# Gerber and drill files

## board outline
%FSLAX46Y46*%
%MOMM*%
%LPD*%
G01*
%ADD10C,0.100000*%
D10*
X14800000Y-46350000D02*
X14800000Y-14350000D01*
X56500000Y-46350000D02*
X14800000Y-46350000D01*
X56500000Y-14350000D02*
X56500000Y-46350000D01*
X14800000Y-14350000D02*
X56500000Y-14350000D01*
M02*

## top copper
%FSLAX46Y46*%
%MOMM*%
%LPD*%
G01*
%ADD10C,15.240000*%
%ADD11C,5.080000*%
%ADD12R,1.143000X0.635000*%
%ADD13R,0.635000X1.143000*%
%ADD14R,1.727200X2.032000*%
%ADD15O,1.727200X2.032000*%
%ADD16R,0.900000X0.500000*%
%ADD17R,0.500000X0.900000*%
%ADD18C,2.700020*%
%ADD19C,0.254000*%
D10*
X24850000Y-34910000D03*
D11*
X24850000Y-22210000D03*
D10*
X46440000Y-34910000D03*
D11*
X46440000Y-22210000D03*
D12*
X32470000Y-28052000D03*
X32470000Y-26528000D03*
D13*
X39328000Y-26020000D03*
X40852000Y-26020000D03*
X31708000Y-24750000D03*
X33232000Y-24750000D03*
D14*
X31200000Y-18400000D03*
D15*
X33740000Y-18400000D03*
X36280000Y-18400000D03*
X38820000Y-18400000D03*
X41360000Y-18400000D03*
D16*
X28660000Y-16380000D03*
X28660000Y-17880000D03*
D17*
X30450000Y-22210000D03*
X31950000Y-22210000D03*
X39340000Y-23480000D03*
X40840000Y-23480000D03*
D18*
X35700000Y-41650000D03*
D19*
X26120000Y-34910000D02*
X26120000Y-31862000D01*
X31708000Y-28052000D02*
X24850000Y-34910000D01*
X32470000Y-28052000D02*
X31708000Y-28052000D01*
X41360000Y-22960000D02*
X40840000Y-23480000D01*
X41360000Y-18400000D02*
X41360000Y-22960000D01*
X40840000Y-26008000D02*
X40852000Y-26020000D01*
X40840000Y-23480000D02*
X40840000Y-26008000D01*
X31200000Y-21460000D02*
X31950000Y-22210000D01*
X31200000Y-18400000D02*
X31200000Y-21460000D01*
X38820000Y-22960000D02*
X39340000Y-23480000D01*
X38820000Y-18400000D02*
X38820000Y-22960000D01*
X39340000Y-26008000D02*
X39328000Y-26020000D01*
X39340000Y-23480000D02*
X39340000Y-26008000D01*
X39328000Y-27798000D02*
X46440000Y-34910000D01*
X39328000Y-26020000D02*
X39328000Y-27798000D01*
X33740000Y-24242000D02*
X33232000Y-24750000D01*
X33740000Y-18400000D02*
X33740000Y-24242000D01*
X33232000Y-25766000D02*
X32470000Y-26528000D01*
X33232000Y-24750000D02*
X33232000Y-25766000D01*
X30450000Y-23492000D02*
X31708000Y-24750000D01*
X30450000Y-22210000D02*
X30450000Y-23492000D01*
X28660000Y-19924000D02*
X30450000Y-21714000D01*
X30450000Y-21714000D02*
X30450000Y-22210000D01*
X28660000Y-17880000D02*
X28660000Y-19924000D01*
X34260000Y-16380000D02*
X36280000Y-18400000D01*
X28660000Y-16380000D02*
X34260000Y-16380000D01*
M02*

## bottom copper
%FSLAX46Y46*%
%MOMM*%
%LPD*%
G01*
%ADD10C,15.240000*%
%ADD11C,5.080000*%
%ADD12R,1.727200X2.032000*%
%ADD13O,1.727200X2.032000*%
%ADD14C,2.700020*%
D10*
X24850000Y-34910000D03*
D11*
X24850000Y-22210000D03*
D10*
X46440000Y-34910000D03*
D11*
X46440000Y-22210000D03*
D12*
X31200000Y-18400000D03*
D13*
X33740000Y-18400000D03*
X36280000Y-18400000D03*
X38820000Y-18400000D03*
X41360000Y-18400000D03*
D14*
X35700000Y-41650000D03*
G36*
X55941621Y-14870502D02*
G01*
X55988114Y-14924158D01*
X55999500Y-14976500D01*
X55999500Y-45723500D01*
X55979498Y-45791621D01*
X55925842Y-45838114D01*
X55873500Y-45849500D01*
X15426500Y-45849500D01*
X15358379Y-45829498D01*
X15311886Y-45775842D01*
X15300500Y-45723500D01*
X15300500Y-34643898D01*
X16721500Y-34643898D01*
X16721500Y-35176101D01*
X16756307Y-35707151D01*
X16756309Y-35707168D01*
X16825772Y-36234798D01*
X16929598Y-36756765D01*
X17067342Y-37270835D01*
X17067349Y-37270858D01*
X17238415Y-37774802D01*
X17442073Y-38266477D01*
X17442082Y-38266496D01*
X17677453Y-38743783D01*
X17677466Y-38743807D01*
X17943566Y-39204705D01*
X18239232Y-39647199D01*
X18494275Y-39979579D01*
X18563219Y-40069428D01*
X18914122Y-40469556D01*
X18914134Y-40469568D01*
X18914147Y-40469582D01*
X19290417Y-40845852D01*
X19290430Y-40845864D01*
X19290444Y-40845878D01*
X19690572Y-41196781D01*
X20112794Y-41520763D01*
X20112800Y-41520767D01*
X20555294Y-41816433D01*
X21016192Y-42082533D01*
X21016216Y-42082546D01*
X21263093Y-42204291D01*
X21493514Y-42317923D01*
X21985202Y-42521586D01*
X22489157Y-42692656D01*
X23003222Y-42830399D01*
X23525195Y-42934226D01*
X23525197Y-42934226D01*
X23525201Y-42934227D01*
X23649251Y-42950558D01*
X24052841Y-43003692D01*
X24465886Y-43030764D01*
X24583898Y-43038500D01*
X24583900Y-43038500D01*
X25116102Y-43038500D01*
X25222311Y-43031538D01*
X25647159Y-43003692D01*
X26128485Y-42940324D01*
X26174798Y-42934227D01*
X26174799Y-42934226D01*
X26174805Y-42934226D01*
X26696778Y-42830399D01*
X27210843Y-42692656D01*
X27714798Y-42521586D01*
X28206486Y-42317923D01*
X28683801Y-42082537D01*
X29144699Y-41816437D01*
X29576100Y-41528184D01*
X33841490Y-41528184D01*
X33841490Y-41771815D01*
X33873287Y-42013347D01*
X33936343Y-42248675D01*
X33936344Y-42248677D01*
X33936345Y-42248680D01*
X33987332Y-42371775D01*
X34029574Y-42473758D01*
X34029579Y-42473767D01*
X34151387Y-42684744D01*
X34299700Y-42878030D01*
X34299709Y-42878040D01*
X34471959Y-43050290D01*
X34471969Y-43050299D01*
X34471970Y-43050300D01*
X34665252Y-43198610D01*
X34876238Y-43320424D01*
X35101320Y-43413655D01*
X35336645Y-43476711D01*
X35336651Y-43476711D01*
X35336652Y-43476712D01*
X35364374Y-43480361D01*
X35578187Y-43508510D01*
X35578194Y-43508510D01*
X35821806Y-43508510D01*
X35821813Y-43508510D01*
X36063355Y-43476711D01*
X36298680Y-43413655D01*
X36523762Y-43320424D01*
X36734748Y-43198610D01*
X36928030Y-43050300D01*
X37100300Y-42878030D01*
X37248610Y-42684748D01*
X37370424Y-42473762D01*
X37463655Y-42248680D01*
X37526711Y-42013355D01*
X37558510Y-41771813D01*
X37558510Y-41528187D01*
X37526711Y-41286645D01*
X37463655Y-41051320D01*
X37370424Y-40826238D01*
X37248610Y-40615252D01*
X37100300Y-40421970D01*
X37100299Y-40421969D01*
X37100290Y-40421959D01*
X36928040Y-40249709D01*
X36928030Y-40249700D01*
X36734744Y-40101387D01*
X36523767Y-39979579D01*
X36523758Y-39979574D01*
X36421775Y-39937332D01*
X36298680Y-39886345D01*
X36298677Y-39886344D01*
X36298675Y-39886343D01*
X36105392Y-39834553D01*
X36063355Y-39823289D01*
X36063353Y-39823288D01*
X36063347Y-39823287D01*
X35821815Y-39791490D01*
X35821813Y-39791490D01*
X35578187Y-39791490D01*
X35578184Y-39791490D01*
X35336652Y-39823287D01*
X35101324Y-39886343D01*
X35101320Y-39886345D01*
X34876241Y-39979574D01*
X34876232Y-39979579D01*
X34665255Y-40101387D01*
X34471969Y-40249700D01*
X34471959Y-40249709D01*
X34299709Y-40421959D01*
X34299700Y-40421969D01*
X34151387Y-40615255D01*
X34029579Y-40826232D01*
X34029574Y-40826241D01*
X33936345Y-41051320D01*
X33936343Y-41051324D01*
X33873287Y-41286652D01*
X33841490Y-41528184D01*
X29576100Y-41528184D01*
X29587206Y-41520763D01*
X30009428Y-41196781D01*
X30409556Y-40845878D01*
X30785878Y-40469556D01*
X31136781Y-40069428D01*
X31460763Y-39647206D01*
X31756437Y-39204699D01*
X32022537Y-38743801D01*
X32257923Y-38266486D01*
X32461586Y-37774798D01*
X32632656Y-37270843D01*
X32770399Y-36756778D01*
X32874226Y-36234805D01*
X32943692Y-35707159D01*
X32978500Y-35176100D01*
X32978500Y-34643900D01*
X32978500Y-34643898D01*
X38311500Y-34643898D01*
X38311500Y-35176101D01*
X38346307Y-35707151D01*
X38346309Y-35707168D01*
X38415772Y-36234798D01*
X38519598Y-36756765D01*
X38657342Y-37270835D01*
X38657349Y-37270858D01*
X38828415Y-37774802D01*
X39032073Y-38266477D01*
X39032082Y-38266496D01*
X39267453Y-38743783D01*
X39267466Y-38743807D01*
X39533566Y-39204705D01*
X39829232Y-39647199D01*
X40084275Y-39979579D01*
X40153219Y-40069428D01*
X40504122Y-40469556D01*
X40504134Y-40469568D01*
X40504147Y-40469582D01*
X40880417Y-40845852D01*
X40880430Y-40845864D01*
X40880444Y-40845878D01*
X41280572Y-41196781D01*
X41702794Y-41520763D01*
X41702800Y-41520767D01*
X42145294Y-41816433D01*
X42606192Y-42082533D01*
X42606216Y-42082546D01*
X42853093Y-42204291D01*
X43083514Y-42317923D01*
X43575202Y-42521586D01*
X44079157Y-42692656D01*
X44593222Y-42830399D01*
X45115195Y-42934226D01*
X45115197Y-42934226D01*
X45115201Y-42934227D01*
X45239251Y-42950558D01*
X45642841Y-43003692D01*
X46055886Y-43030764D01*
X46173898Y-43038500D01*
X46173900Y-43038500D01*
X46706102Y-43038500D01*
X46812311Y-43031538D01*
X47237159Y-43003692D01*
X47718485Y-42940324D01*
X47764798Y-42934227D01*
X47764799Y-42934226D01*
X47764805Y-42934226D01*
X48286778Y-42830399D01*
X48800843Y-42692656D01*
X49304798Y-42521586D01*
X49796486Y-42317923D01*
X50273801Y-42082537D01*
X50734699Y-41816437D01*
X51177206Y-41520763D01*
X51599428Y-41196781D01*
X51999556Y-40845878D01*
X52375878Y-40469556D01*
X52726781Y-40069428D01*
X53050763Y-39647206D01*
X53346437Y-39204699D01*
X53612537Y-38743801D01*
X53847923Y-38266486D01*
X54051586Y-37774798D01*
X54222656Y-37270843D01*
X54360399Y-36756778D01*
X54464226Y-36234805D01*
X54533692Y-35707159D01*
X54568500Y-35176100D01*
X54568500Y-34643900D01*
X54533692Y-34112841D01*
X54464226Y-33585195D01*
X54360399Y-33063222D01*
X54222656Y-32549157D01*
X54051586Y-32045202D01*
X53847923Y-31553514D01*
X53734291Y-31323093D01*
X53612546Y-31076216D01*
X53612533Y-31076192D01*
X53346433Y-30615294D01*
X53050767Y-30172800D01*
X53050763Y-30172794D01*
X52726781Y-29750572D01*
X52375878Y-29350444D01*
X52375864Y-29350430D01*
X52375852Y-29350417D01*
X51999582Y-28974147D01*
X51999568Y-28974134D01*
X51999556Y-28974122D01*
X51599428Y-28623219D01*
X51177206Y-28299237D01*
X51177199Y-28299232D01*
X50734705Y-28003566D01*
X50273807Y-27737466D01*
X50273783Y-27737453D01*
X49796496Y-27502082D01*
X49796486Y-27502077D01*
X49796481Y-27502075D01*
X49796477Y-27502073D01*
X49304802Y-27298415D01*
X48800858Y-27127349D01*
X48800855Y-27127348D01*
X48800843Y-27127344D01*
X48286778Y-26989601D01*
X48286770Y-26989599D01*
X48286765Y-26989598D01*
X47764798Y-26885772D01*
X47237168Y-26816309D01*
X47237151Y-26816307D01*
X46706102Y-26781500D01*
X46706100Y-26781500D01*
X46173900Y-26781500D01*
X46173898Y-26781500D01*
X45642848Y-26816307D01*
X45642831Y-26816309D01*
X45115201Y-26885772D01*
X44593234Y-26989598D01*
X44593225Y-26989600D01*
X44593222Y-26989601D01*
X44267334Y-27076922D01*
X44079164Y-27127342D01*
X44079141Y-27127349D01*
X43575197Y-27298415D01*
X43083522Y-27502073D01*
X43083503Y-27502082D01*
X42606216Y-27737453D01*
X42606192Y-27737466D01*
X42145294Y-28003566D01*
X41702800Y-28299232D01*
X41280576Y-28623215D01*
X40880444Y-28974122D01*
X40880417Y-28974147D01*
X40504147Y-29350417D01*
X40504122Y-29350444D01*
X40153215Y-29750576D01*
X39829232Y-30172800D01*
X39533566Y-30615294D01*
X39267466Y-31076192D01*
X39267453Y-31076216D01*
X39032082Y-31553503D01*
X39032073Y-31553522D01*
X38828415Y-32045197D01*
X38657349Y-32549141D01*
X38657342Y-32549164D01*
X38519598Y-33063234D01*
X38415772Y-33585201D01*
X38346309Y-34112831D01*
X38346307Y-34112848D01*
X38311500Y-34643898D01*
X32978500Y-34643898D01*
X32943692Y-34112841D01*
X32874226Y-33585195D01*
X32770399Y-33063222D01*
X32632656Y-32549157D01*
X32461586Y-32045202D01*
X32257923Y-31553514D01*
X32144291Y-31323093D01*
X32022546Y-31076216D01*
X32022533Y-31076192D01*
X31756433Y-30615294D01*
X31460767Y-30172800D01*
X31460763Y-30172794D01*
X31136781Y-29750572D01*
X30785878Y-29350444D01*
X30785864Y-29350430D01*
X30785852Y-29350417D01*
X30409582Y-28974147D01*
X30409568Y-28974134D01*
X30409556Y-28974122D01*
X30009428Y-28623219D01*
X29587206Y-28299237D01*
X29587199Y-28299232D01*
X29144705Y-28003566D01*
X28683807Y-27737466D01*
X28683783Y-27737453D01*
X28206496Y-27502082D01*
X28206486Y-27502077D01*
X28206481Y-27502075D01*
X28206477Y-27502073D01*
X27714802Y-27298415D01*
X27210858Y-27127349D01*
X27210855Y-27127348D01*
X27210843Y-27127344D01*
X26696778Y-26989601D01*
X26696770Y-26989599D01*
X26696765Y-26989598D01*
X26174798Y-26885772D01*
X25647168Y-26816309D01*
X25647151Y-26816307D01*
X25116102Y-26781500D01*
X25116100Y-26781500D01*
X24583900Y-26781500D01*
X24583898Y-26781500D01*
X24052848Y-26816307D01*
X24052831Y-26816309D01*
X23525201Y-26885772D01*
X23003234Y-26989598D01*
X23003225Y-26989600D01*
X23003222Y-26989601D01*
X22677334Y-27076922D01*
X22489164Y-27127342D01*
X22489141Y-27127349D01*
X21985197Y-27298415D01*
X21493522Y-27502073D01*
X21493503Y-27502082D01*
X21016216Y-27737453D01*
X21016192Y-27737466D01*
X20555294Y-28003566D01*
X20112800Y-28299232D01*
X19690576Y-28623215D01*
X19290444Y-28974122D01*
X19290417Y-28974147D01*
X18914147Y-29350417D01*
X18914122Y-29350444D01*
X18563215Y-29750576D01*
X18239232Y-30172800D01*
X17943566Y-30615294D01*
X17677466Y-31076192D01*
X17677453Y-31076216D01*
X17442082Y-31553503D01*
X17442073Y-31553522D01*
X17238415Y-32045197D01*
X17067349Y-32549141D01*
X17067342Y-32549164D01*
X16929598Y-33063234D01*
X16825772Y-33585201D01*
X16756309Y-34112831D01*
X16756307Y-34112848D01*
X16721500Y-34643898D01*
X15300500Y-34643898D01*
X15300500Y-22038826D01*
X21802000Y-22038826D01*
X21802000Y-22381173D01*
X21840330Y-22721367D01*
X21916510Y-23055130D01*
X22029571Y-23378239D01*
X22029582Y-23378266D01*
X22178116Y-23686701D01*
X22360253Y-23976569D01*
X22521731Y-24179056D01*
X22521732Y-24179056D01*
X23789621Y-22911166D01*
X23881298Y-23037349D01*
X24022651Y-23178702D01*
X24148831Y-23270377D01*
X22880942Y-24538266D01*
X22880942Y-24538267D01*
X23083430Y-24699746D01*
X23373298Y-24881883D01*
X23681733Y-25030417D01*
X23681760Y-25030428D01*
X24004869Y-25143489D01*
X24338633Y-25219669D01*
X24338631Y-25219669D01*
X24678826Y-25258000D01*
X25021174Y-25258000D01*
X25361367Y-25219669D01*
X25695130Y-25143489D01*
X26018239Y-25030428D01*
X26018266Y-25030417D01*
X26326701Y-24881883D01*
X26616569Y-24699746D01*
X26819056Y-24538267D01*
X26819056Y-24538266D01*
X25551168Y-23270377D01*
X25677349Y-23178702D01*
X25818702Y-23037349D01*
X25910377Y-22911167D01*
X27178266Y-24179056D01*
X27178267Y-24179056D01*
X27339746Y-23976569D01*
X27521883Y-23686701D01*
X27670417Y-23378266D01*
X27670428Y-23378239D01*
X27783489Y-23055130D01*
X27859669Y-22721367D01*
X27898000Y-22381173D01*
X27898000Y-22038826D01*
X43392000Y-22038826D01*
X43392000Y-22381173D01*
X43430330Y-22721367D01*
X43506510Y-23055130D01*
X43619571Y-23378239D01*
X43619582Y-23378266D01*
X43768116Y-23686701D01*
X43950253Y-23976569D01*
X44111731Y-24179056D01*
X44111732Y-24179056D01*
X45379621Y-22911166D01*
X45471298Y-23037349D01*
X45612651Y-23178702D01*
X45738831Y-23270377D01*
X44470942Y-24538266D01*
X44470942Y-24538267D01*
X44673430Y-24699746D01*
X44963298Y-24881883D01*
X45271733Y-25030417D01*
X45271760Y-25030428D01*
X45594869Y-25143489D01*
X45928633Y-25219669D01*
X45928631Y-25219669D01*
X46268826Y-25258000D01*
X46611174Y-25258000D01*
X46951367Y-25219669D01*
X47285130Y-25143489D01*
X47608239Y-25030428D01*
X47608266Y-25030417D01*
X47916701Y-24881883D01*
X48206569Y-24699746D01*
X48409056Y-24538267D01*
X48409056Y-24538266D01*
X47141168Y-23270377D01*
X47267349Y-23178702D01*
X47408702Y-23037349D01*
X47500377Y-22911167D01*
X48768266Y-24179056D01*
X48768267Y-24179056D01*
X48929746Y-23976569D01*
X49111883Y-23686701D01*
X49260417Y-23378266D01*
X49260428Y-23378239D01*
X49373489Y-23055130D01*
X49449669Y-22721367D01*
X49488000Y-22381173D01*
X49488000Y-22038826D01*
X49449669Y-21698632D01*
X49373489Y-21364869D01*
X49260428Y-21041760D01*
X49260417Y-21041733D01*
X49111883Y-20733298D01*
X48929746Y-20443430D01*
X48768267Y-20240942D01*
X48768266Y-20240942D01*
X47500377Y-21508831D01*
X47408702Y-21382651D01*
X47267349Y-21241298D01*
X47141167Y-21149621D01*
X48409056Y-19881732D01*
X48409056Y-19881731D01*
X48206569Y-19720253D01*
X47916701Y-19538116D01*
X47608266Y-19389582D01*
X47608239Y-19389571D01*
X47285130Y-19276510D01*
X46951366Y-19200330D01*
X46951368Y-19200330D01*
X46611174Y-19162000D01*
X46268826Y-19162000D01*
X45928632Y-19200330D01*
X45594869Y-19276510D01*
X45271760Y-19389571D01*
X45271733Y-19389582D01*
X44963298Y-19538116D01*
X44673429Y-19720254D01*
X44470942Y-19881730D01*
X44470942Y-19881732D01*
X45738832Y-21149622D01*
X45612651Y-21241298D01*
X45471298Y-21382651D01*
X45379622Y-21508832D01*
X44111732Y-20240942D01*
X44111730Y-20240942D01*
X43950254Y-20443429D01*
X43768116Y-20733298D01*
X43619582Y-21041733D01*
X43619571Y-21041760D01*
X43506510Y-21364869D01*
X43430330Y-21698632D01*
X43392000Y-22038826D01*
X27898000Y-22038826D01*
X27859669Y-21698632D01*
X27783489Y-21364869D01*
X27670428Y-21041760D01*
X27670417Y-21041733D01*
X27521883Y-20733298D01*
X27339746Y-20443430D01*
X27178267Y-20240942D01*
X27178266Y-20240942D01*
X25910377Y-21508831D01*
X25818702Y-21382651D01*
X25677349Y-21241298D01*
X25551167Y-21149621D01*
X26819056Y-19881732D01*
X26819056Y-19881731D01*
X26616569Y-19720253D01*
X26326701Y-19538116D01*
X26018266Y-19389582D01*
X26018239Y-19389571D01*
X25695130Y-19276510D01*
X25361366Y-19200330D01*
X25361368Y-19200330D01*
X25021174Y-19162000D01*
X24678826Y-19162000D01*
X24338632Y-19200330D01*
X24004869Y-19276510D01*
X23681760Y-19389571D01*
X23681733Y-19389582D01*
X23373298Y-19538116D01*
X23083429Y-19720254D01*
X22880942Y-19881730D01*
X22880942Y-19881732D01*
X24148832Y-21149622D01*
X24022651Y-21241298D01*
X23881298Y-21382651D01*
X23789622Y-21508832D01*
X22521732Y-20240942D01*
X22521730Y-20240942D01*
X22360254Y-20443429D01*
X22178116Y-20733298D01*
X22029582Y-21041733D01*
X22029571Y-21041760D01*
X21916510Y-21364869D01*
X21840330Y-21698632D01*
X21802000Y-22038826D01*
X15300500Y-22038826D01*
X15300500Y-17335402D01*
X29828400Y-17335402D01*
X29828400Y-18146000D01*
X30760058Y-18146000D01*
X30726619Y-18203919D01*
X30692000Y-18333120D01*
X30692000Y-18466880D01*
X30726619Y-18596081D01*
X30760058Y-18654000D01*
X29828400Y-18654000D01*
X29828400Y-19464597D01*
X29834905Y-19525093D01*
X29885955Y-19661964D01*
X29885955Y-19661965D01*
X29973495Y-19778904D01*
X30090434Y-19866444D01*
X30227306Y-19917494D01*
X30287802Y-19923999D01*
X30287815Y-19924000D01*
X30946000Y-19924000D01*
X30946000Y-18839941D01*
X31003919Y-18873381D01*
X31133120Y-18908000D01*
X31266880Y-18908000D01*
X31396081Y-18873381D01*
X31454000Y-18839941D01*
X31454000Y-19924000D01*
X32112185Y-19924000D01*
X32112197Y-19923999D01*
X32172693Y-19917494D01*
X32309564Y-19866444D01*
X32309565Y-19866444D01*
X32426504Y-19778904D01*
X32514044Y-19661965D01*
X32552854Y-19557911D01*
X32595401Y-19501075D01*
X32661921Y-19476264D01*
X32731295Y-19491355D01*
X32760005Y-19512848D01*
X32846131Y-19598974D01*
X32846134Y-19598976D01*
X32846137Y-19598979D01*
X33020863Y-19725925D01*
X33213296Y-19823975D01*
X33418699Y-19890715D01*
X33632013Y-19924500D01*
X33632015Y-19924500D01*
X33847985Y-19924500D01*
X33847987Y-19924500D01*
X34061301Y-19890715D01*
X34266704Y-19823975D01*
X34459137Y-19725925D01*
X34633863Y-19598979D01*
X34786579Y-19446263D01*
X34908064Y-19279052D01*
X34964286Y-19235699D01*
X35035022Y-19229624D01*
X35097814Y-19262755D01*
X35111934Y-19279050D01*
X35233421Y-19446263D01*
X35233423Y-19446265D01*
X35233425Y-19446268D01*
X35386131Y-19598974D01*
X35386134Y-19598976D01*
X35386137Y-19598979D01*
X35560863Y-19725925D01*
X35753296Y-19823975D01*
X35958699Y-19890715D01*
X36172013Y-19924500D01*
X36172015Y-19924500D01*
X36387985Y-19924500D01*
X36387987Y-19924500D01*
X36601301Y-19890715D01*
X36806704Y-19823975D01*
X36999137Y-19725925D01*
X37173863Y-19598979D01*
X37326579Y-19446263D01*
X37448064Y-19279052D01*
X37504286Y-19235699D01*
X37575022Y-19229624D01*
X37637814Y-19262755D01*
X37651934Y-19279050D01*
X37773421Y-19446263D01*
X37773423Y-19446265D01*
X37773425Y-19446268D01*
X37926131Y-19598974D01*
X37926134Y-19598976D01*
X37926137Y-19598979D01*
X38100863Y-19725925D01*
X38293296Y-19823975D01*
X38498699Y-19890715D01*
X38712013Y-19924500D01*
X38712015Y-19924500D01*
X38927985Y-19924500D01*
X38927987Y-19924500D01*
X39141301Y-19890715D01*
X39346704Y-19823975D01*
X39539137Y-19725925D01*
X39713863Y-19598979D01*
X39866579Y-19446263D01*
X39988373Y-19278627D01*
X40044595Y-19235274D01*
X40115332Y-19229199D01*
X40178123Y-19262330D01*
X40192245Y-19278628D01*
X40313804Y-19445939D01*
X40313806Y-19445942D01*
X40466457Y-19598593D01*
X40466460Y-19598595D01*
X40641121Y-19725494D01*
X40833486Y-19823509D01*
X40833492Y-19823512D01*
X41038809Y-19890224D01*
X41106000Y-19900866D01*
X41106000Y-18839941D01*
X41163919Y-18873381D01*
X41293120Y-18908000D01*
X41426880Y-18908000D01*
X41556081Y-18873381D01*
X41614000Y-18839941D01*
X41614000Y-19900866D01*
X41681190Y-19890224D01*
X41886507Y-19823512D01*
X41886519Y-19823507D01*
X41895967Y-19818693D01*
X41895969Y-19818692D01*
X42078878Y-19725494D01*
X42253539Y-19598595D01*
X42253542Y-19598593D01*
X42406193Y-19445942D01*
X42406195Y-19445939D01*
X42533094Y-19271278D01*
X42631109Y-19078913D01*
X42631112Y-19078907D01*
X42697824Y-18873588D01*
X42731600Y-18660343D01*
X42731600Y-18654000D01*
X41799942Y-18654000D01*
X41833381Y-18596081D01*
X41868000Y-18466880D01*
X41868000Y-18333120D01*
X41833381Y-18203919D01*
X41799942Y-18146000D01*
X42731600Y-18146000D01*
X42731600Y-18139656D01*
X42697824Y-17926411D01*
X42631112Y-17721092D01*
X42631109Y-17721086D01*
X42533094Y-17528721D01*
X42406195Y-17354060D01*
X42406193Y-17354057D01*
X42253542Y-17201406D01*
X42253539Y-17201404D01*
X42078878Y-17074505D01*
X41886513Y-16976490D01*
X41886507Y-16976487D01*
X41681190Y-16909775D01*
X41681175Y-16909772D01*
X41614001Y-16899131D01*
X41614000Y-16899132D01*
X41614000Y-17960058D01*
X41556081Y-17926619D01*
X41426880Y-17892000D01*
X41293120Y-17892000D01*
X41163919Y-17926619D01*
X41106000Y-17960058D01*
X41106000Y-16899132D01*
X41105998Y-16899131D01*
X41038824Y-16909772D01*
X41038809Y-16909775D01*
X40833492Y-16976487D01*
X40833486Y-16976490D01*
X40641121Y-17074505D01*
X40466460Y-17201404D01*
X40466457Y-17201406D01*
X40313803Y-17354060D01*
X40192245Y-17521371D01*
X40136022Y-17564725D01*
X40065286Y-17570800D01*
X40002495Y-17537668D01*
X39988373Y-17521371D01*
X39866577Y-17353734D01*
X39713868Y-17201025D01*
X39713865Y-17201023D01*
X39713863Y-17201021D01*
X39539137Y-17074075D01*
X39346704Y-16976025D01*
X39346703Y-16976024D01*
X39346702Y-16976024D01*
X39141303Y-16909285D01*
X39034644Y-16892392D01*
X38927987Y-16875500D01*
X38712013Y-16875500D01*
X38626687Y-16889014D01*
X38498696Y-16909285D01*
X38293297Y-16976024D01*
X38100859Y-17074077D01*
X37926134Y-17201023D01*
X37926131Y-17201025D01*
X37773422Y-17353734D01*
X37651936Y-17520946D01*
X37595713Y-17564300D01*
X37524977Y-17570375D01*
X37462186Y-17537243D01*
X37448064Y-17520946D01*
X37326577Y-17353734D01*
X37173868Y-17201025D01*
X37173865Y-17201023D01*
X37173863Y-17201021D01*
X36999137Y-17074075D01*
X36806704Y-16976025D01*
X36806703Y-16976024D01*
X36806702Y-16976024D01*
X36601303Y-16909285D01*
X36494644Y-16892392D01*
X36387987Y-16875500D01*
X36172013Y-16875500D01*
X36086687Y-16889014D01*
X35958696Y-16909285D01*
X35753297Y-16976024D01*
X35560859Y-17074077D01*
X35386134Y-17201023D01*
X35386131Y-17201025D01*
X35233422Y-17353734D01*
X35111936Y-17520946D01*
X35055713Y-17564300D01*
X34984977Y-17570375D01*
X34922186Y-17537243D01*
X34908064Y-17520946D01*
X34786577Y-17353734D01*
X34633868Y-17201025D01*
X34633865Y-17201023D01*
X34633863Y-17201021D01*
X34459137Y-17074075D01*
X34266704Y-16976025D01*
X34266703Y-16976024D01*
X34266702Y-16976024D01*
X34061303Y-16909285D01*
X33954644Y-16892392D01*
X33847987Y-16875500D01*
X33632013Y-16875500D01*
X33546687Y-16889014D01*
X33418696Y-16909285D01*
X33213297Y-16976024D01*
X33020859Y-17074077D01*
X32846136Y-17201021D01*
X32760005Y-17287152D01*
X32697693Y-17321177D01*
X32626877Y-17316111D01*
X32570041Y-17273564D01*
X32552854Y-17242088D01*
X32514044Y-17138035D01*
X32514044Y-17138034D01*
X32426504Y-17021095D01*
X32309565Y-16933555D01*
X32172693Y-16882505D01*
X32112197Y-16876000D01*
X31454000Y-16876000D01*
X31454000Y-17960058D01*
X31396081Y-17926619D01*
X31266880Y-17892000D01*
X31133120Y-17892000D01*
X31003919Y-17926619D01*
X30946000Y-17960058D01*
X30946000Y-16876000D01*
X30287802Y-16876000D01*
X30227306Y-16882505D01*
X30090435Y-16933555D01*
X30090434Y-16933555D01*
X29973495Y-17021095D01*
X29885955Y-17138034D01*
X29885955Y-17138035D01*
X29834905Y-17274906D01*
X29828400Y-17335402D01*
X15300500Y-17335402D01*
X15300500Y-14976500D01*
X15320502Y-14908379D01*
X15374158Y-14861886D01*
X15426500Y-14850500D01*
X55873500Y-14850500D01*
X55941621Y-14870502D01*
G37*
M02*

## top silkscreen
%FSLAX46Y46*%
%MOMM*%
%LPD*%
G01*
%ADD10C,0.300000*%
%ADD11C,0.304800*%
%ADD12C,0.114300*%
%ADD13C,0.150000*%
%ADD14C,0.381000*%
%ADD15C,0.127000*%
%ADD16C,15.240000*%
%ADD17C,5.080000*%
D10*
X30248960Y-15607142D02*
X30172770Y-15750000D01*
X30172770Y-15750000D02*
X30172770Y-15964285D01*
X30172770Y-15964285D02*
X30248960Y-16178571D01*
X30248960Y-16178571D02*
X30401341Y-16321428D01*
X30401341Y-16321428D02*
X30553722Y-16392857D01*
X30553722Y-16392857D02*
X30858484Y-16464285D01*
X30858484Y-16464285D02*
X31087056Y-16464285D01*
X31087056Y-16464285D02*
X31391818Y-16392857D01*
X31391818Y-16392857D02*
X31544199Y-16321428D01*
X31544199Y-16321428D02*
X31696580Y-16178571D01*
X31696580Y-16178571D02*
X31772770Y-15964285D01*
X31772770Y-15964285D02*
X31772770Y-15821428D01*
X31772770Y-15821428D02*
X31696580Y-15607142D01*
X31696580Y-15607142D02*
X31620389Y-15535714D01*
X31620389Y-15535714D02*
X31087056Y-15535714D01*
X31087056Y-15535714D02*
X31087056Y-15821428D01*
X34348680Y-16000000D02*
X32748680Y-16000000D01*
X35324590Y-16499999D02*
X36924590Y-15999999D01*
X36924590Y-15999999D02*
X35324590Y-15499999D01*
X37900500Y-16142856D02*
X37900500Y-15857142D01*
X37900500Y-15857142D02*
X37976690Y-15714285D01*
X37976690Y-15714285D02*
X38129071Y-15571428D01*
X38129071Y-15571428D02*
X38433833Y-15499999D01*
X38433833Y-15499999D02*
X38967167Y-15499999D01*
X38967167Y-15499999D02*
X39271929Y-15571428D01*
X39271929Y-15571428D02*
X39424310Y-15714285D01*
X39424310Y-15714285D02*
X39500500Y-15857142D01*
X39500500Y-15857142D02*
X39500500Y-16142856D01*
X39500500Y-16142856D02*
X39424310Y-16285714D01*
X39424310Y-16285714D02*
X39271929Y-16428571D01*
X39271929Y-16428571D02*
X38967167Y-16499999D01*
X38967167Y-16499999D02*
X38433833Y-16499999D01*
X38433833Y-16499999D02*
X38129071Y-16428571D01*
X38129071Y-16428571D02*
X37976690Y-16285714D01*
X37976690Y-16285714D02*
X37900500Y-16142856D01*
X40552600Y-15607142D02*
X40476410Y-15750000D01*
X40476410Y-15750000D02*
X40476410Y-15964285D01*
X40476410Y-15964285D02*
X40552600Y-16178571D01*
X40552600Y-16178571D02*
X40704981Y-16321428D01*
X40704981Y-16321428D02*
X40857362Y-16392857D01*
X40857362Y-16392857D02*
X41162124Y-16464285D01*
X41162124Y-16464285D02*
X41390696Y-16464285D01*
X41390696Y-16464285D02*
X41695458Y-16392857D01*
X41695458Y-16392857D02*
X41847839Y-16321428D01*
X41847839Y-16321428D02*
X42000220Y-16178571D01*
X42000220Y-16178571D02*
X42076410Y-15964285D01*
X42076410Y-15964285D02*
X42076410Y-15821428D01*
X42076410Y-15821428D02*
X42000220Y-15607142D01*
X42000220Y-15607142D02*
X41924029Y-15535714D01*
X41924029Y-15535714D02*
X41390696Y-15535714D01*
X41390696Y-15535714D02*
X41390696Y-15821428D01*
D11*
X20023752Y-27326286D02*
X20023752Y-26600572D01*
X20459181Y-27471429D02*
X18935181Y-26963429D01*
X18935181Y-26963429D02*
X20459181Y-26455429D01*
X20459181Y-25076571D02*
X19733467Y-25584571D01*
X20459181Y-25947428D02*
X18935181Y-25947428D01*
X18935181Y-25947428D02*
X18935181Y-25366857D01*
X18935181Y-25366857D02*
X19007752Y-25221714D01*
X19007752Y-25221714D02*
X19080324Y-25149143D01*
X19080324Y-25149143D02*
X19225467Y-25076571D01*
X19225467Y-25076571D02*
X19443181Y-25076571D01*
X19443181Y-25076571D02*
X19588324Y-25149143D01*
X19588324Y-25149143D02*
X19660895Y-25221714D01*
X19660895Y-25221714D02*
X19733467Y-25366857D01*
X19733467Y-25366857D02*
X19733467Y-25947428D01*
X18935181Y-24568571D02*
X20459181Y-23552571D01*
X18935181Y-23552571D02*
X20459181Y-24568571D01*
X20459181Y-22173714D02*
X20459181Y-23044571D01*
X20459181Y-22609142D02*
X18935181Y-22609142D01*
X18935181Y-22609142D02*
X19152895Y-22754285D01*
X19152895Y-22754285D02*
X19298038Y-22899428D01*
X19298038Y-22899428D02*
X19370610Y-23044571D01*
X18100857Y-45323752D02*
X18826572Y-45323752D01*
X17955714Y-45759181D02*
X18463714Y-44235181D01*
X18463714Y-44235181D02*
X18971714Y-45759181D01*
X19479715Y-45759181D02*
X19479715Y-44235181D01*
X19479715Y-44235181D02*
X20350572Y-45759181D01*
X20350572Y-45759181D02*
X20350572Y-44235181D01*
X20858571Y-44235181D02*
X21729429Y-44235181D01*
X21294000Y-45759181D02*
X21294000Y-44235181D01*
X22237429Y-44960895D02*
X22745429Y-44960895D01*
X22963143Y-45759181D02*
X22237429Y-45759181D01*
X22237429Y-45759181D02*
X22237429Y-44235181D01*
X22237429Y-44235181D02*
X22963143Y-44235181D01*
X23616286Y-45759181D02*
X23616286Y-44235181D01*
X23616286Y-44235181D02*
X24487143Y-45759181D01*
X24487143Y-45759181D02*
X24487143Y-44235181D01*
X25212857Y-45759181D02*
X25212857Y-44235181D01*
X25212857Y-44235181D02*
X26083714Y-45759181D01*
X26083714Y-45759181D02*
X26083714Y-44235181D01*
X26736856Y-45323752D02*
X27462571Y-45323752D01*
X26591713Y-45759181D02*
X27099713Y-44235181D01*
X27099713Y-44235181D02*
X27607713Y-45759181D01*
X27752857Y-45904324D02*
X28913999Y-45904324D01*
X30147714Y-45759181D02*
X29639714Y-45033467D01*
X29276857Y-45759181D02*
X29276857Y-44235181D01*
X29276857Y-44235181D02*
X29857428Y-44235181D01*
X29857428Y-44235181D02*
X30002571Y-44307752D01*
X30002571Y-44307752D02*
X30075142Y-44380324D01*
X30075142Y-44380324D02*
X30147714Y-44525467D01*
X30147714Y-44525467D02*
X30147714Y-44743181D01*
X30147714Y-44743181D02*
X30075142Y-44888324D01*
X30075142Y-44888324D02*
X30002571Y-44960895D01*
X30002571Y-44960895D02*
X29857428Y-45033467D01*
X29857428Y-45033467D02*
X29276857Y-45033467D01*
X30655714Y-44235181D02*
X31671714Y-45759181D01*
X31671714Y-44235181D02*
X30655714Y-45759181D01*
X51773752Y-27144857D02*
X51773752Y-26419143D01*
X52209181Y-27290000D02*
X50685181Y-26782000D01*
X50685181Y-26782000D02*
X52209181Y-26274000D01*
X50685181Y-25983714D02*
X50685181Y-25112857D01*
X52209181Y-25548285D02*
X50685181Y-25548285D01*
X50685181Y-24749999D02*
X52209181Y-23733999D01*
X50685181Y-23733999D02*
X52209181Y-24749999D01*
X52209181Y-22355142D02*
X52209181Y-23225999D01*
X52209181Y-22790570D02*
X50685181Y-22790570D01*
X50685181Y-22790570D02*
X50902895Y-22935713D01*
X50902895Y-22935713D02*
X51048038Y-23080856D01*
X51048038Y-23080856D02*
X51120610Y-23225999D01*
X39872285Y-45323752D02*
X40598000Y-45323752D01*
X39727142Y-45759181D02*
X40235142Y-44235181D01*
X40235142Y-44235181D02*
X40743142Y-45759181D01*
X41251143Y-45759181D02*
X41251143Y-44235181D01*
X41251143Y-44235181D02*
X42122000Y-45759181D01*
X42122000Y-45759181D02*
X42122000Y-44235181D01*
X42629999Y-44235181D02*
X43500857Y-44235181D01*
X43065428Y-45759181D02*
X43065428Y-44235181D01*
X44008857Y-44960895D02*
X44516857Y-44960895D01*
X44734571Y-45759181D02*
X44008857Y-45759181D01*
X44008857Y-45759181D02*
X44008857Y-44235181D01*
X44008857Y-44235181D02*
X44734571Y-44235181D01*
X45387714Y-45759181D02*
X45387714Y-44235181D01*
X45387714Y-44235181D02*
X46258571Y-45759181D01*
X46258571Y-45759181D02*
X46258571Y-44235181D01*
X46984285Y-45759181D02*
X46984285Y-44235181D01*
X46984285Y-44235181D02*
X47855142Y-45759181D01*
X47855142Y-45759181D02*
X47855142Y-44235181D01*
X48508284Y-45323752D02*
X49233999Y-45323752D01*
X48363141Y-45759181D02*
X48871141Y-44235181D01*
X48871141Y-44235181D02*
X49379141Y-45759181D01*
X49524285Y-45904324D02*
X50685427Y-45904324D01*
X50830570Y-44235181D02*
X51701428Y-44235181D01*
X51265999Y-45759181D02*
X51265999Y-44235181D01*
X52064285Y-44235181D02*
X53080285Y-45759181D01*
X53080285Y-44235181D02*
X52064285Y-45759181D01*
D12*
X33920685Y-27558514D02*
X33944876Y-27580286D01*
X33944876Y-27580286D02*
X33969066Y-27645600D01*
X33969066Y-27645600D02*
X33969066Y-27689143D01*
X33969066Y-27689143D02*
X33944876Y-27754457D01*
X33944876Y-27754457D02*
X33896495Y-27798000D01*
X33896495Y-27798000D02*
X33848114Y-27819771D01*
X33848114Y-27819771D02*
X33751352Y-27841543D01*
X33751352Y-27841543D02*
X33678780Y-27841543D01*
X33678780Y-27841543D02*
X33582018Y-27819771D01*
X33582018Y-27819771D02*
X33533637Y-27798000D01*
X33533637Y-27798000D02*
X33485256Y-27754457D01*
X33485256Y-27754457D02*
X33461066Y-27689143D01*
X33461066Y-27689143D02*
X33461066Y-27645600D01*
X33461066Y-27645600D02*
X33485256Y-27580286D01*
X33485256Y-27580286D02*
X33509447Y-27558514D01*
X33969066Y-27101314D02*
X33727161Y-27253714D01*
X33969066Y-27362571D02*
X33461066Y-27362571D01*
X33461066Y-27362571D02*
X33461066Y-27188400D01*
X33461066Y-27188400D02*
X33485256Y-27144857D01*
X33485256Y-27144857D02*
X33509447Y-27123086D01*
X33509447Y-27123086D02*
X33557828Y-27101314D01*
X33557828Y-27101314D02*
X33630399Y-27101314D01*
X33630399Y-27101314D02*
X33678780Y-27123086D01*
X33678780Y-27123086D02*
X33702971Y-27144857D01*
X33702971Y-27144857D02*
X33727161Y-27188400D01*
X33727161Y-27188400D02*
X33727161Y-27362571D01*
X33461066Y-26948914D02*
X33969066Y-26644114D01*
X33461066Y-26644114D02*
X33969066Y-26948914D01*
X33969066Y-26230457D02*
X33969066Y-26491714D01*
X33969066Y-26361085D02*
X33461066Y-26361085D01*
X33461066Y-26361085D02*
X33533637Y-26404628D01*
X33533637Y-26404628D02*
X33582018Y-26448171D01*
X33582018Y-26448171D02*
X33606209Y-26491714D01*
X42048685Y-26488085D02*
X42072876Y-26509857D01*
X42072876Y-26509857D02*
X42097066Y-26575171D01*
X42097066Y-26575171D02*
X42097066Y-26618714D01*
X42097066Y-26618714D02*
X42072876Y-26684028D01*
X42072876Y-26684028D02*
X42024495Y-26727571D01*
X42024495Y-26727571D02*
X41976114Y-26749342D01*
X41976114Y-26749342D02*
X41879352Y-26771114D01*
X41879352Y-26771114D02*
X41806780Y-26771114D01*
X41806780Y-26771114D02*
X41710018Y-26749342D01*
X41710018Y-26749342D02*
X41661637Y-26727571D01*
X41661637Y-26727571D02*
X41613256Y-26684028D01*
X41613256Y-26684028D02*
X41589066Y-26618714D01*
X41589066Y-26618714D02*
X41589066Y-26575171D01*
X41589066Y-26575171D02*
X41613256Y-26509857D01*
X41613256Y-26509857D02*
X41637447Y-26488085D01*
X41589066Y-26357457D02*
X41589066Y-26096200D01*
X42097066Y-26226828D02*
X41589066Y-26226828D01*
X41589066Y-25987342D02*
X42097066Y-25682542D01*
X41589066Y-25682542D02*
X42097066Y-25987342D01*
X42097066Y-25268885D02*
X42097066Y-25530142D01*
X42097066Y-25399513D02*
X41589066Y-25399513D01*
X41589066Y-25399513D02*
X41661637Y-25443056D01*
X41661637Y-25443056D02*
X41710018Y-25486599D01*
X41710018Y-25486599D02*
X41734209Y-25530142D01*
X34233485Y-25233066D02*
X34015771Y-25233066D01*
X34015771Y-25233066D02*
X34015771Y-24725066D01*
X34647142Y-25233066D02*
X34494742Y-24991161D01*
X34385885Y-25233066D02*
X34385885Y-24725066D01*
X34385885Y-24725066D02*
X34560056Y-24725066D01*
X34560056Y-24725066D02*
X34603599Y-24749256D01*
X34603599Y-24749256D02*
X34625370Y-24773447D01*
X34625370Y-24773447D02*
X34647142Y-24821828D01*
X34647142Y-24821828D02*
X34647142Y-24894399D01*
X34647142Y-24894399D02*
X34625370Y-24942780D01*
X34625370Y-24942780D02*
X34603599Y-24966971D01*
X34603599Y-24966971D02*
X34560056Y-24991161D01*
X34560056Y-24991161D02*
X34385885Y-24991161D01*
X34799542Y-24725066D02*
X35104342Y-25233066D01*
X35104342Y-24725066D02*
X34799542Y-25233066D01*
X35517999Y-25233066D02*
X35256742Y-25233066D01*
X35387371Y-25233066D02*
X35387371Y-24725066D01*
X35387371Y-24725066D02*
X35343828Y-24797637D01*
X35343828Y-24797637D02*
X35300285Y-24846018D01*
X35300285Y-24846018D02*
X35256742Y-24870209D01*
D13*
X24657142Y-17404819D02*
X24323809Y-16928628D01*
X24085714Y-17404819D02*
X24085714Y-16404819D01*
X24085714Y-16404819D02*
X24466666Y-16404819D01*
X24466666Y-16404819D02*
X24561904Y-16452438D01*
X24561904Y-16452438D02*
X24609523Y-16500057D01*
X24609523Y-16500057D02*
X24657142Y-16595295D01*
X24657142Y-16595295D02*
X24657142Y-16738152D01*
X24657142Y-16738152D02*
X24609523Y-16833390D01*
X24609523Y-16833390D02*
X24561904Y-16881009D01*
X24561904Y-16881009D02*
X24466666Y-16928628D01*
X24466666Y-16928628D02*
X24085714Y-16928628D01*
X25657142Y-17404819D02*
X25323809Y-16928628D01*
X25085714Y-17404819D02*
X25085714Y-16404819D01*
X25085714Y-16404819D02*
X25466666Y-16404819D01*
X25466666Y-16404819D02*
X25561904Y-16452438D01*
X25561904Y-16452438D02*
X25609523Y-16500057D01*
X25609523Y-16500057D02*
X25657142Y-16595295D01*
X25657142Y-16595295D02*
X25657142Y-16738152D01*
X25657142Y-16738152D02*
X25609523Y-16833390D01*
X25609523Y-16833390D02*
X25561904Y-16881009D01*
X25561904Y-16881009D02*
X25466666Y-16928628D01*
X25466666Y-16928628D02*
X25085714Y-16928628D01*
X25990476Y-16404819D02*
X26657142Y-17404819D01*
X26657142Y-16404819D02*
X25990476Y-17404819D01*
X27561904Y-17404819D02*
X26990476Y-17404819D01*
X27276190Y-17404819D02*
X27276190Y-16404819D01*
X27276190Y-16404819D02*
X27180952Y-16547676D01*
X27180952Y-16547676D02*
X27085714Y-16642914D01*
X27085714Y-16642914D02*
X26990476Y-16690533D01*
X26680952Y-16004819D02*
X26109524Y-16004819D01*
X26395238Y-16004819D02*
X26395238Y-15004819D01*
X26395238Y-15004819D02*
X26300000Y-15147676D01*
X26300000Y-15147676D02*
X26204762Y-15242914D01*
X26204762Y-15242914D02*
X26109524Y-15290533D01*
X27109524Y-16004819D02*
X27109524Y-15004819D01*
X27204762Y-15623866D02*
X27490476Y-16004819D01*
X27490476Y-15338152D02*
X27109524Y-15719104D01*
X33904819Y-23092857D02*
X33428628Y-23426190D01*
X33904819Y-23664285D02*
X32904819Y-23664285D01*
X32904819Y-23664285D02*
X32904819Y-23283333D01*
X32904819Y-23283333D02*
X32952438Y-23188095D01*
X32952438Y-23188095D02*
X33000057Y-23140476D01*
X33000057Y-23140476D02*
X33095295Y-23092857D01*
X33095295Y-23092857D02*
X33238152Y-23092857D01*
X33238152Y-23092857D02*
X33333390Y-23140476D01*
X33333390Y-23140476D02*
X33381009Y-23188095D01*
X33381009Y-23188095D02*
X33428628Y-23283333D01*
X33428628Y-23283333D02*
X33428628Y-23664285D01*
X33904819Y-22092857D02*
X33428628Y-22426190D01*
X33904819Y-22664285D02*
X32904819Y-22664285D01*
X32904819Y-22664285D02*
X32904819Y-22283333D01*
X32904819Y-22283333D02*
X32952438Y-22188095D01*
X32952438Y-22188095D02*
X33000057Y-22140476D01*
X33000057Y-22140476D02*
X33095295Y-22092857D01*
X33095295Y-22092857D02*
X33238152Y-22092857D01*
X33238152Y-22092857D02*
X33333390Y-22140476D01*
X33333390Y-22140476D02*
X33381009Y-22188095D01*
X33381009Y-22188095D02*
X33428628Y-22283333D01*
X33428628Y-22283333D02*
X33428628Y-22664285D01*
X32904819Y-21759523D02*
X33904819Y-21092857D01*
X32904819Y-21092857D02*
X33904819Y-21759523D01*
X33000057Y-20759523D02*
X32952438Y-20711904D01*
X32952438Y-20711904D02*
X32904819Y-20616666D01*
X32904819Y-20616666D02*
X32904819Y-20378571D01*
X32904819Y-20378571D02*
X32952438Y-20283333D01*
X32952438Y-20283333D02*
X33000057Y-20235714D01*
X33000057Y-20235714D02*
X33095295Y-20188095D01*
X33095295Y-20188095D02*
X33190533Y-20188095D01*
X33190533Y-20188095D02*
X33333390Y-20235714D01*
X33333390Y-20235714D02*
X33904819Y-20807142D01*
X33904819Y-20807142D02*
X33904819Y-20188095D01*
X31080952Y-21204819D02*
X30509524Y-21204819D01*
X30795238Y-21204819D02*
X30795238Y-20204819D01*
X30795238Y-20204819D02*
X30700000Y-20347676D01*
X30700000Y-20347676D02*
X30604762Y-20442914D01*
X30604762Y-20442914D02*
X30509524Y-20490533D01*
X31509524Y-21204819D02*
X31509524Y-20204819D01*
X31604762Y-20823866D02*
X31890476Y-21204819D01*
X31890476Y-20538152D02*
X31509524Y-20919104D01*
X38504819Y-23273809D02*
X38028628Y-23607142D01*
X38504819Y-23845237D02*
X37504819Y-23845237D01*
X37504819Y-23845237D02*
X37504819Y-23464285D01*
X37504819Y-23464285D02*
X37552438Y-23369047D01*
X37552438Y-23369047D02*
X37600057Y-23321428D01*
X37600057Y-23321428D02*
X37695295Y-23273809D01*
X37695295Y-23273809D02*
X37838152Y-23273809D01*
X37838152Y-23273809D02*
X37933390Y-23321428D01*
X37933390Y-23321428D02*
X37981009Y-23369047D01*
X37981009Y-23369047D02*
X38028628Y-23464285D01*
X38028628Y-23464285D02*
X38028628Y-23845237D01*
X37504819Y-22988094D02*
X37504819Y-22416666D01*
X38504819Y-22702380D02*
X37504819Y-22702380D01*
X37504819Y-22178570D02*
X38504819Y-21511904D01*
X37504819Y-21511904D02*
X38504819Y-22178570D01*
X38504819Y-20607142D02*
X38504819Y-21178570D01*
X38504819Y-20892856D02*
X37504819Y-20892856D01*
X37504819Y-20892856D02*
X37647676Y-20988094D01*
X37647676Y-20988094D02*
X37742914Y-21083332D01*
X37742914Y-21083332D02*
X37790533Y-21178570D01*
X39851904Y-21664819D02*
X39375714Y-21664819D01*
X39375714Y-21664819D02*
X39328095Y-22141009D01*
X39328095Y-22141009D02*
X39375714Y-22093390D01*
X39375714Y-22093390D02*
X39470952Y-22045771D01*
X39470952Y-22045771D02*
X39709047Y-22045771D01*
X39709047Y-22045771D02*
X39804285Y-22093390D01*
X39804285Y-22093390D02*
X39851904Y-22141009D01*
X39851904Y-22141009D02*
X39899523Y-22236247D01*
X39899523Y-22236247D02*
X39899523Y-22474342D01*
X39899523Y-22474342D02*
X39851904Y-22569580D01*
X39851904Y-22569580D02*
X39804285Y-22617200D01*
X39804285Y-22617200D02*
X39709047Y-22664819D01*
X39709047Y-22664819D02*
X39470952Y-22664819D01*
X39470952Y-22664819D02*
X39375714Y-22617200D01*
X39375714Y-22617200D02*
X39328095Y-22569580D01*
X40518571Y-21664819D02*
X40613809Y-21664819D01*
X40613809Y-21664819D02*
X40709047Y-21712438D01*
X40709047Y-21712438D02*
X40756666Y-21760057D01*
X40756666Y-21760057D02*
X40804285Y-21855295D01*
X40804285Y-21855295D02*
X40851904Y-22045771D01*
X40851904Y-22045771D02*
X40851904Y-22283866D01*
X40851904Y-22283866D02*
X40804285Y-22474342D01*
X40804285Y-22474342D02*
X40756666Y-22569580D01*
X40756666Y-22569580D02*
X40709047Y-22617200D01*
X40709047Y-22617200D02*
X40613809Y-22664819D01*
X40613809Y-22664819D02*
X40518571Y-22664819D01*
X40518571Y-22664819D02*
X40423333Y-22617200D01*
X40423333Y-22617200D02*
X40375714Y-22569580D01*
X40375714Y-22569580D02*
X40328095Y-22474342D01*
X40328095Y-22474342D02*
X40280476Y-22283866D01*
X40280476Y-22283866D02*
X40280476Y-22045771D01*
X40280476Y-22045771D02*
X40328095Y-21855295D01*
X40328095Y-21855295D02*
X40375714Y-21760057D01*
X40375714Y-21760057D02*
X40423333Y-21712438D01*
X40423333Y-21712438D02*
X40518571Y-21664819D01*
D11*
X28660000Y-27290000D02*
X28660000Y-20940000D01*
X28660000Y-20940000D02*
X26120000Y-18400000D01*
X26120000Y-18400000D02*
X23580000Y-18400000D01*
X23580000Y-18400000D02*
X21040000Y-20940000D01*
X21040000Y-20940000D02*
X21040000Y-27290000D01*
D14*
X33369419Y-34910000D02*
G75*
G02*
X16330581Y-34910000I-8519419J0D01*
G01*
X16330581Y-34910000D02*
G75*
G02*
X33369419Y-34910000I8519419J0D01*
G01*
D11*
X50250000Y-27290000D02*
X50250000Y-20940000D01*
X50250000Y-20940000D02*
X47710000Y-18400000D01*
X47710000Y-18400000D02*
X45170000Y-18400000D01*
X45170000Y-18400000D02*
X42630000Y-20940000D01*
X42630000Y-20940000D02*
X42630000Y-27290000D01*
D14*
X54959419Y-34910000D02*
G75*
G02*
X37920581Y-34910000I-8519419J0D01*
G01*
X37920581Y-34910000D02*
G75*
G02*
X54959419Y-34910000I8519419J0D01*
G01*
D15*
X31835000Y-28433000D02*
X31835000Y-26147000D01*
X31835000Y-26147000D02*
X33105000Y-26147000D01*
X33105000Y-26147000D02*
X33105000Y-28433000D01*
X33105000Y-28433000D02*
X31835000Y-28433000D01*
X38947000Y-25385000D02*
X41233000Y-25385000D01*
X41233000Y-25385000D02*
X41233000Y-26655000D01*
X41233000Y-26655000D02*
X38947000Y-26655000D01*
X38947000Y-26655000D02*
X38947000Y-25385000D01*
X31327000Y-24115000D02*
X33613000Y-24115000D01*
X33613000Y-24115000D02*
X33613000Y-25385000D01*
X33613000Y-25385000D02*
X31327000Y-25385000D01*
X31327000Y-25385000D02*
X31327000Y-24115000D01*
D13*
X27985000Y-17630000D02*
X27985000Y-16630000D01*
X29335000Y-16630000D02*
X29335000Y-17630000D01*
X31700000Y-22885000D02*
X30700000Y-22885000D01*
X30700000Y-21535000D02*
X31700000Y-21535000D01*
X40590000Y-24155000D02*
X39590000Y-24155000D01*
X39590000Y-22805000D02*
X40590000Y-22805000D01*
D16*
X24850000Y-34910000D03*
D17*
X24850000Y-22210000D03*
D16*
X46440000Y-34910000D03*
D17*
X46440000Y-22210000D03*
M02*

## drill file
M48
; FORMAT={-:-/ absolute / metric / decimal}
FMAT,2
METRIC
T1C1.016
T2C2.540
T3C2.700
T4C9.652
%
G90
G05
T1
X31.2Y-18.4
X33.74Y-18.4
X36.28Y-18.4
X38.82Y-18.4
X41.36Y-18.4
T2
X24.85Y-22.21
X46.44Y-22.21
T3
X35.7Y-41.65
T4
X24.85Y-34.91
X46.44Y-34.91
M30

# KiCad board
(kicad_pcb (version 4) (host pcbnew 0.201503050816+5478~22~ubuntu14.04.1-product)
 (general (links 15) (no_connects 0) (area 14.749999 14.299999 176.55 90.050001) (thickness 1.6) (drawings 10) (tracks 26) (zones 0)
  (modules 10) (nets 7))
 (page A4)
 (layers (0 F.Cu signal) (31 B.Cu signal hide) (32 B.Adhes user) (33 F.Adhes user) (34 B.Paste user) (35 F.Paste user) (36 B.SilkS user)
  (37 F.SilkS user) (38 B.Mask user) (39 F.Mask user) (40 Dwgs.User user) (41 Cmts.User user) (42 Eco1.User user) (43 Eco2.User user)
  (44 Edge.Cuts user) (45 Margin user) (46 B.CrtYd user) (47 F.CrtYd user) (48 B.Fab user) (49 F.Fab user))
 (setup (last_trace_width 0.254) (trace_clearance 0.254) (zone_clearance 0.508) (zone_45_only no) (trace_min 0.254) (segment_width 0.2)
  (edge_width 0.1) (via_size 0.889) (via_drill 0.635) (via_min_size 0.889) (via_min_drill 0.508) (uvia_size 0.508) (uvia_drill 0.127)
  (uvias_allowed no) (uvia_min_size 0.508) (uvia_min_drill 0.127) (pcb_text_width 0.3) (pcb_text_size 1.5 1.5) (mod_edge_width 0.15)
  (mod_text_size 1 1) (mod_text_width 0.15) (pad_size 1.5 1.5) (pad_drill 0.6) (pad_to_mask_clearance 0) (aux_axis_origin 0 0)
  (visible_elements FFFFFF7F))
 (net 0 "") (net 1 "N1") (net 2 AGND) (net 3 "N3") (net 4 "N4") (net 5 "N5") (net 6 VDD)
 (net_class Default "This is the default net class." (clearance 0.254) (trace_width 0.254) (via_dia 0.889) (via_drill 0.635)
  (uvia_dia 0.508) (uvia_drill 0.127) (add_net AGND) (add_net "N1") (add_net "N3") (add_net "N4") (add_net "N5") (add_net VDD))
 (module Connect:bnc (layer F.Cu) (at 24.85 34.91 90)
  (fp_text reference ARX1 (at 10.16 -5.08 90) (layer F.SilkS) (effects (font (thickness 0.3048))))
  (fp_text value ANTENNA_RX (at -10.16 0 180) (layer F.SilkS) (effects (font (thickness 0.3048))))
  (fp_line (start 7.62 3.81) (end 13.97 3.81) (layer F.SilkS) (width 0.3048))
  (fp_line (start 13.97 3.81) (end 16.51 1.27) (layer F.SilkS) (width 0.3048))
  (fp_line (start 16.51 1.27) (end 16.51 -1.27) (layer F.SilkS) (width 0.3048))
  (fp_line (start 16.51 -1.27) (end 13.97 -3.81) (layer F.SilkS) (width 0.3048))
  (fp_line (start 13.97 -3.81) (end 7.62 -3.81) (layer F.SilkS) (width 0.3048))
  (fp_circle (center 0 0) (end 7.62 3.81) (layer F.SilkS) (width 0.381))
  (pad 2 thru_hole circle (at 0 0 90) (size 15.24 15.24) (drill 9.652) (layers *.Cu *.Mask F.SilkS) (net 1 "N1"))
  (pad 1 thru_hole circle (at 12.7 0 90) (size 5.08 5.08) (drill 2.54) (layers *.Cu *.Mask F.SilkS) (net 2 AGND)))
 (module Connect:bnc (layer F.Cu) (at 46.44 34.91 90)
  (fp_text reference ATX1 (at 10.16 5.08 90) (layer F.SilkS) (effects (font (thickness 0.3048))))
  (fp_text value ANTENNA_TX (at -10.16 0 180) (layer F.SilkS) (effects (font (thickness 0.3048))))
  (fp_line (start 7.62 3.81) (end 13.97 3.81) (layer F.SilkS) (width 0.3048))
  (fp_line (start 13.97 3.81) (end 16.51 1.27) (layer F.SilkS) (width 0.3048))
  (fp_line (start 16.51 1.27) (end 16.51 -1.27) (layer F.SilkS) (width 0.3048))
  (fp_line (start 16.51 -1.27) (end 13.97 -3.81) (layer F.SilkS) (width 0.3048))
  (fp_line (start 13.97 -3.81) (end 7.62 -3.81) (layer F.SilkS) (width 0.3048))
  (fp_circle (center 0 0) (end 7.62 3.81) (layer F.SilkS) (width 0.381))
  (pad 2 thru_hole circle (at 0 0 90) (size 15.24 15.24) (drill 9.652) (layers *.Cu *.Mask F.SilkS) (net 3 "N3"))
  (pad 1 thru_hole circle (at 12.7 0 90) (size 5.08 5.08) (drill 2.54) (layers *.Cu *.Mask F.SilkS) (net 2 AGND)))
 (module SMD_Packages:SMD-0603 (layer F.Cu) (at 32.47 27.29 90)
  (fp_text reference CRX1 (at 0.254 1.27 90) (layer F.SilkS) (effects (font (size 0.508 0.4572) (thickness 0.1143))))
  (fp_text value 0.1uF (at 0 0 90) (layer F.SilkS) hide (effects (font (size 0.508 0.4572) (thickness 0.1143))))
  (fp_line (start -1.143 -0.635) (end 1.143 -0.635) (layer F.SilkS) (width 0.127))
  (fp_line (start 1.143 -0.635) (end 1.143 0.635) (layer F.SilkS) (width 0.127))
  (fp_line (start 1.143 0.635) (end -1.143 0.635) (layer F.SilkS) (width 0.127))
  (fp_line (start -1.143 0.635) (end -1.143 -0.635) (layer F.SilkS) (width 0.127))
  (pad 1 smd rect (at -0.762 0 90) (size 0.635 1.143) (layers F.Cu F.Paste F.Mask) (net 1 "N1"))
  (pad 2 smd rect (at 0.762 0 90) (size 0.635 1.143) (layers F.Cu F.Paste F.Mask) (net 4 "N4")))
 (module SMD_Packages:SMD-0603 (layer F.Cu) (at 40.09 26.02)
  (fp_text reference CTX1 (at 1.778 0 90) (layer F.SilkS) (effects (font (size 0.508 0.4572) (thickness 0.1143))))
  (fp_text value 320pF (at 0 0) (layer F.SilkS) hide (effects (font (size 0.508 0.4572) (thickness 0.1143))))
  (fp_line (start -1.143 -0.635) (end 1.143 -0.635) (layer F.SilkS) (width 0.127))
  (fp_line (start 1.143 -0.635) (end 1.143 0.635) (layer F.SilkS) (width 0.127))
  (fp_line (start 1.143 0.635) (end -1.143 0.635) (layer F.SilkS) (width 0.127))
  (fp_line (start -1.143 0.635) (end -1.143 -0.635) (layer F.SilkS) (width 0.127))
  (pad 1 smd rect (at -0.762 0) (size 0.635 1.143) (layers F.Cu F.Paste F.Mask) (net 3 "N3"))
  (pad 2 smd rect (at 0.762 0) (size 0.635 1.143) (layers F.Cu F.Paste F.Mask) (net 2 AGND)))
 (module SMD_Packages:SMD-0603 (layer F.Cu) (at 32.47 24.75)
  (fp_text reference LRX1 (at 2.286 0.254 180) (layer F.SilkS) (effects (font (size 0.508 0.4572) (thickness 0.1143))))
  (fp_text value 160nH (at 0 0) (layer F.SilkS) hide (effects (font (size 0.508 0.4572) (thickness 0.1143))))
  (fp_line (start -1.143 -0.635) (end 1.143 -0.635) (layer F.SilkS) (width 0.127))
  (fp_line (start 1.143 -0.635) (end 1.143 0.635) (layer F.SilkS) (width 0.127))
  (fp_line (start 1.143 0.635) (end -1.143 0.635) (layer F.SilkS) (width 0.127))
  (fp_line (start -1.143 0.635) (end -1.143 -0.635) (layer F.SilkS) (width 0.127))
  (pad 1 smd rect (at -0.762 0) (size 0.635 1.143) (layers F.Cu F.Paste F.Mask) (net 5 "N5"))
  (pad 2 smd rect (at 0.762 0) (size 0.635 1.143) (layers F.Cu F.Paste F.Mask) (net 4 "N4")))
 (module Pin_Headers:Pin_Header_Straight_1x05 (layer B.Cu) (at 36.28 18.4)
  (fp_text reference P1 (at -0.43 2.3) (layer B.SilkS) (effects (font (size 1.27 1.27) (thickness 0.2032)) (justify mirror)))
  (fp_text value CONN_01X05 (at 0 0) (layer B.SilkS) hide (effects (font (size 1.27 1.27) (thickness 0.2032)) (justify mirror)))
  (pad 1 thru_hole rect (at -5.08 0) (size 1.7272 2.032) (drill 1.016) (layers *.Cu *.Mask B.SilkS) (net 2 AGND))
  (pad 2 thru_hole oval (at -2.54 0) (size 1.7272 2.032) (drill 1.016) (layers *.Cu *.Mask B.SilkS) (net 4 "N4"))
  (pad 3 thru_hole oval (at 0 0) (size 1.7272 2.032) (drill 1.016) (layers *.Cu *.Mask B.SilkS) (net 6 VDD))
  (pad 4 thru_hole oval (at 2.54 0) (size 1.7272 2.032) (drill 1.016) (layers *.Cu *.Mask B.SilkS) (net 3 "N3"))
  (pad 5 thru_hole oval (at 5.08 0) (size 1.7272 2.032) (drill 1.016) (layers *.Cu *.Mask B.SilkS) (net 2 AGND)))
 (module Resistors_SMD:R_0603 (layer F.Cu) (at 28.66 17.13 270)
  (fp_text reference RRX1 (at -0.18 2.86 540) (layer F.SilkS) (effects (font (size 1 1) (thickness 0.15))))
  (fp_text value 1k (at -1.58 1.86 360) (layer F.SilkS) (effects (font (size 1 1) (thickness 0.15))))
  (fp_line (start 0.5 0.675) (end -0.5 0.675) (layer F.SilkS) (width 0.15))
  (fp_line (start -0.5 -0.675) (end 0.5 -0.675) (layer F.SilkS) (width 0.15))
  (pad 1 smd rect (at -0.75 0 270) (size 0.5 0.9) (layers F.Cu F.Paste F.Mask) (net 6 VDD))
  (pad 2 smd rect (at 0.75 0 270) (size 0.5 0.9) (layers F.Cu F.Paste F.Mask) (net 5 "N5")))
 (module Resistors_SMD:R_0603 (layer F.Cu) (at 31.2 22.21)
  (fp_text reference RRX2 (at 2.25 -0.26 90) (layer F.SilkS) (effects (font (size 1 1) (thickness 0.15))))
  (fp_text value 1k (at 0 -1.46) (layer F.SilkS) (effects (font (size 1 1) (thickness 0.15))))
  (fp_line (start 0.5 0.675) (end -0.5 0.675) (layer F.SilkS) (width 0.15))
  (fp_line (start -0.5 -0.675) (end 0.5 -0.675) (layer F.SilkS) (width 0.15))
  (pad 1 smd rect (at -0.75 0) (size 0.5 0.9) (layers F.Cu F.Paste F.Mask) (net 5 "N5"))
  (pad 2 smd rect (at 0.75 0) (size 0.5 0.9) (layers F.Cu F.Paste F.Mask) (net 2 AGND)))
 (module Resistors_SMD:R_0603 (layer F.Cu) (at 40.09 23.48)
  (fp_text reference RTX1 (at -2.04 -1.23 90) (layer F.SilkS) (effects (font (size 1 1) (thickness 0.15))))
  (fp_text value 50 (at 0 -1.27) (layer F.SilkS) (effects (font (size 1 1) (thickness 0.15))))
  (fp_line (start 0.5 0.675) (end -0.5 0.675) (layer F.SilkS) (width 0.15))
  (fp_line (start -0.5 -0.675) (end 0.5 -0.675) (layer F.SilkS) (width 0.15))
  (pad 1 smd rect (at -0.75 0) (size 0.5 0.9) (layers F.Cu F.Paste F.Mask) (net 3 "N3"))
  (pad 2 smd rect (at 0.75 0) (size 0.5 0.9) (layers F.Cu F.Paste F.Mask) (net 2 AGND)))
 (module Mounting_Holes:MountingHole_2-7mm (layer F.Cu) (at 35.7 41.65)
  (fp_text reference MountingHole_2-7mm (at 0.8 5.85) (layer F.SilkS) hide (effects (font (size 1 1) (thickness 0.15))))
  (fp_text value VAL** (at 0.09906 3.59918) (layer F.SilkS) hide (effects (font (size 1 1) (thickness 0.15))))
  (pad 1 thru_hole circle (at 0 0) (size 2.70002 2.70002) (drill 2.70002) (layers)))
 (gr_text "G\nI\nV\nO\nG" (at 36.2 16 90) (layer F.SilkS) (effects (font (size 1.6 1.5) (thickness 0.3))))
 (gr_line (start 14.8 46.35) (end 14.8 14.35) (angle 90) (layer Edge.Cuts) (width 0.1))
 (gr_line (start 56.5 46.35) (end 14.8 46.35) (angle 90) (layer Edge.Cuts) (width 0.1))
 (gr_line (start 56.5 14.35) (end 56.5 46.35) (angle 90) (layer Edge.Cuts) (width 0.1))
 (gr_line (start 14.8 14.35) (end 56.5 14.35) (angle 90) (layer Edge.Cuts) (width 0.1))
 (segment (start 26.12 34.91) (end 26.12 31.862) (width 0.254) (layer F.Cu) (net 1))
 (segment (start 31.708 28.052) (end 24.85 34.91) (width 0.254) (layer F.Cu) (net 1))
 (segment (start 32.47 28.052) (end 31.708 28.052) (width 0.254) (layer F.Cu) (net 1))
 (segment (start 41.36 22.96) (end 40.84 23.48) (width 0.254) (layer F.Cu) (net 2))
 (segment (start 41.36 18.4) (end 41.36 22.96) (width 0.254) (layer F.Cu) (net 2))
 (segment (start 40.84 26.008) (end 40.852 26.02) (width 0.254) (layer F.Cu) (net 2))
 (segment (start 40.84 23.48) (end 40.84 26.008) (width 0.254) (layer F.Cu) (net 2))
 (segment (start 31.2 21.46) (end 31.95 22.21) (width 0.254) (layer F.Cu) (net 2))
 (segment (start 31.2 18.4) (end 31.2 21.46) (width 0.254) (layer F.Cu) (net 2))
 (segment (start 38.82 22.96) (end 39.34 23.48) (width 0.254) (layer F.Cu) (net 3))
 (segment (start 38.82 18.4) (end 38.82 22.96) (width 0.254) (layer F.Cu) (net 3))
 (segment (start 39.34 26.008) (end 39.328 26.02) (width 0.254) (layer F.Cu) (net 3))
 (segment (start 39.34 23.48) (end 39.34 26.008) (width 0.254) (layer F.Cu) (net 3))
 (segment (start 39.328 27.798) (end 46.44 34.91) (width 0.254) (layer F.Cu) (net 3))
 (segment (start 39.328 26.02) (end 39.328 27.798) (width 0.254) (layer F.Cu) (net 3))
 (segment (start 33.74 24.242) (end 33.232 24.75) (width 0.254) (layer F.Cu) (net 4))
 (segment (start 33.74 18.4) (end 33.74 24.242) (width 0.254) (layer F.Cu) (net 4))
 (segment (start 33.232 25.766) (end 32.47 26.528) (width 0.254) (layer F.Cu) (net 4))
 (segment (start 33.232 24.75) (end 33.232 25.766) (width 0.254) (layer F.Cu) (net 4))
 (segment (start 30.45 23.492) (end 31.708 24.75) (width 0.254) (layer F.Cu) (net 5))
 (segment (start 30.45 22.21) (end 30.45 23.492) (width 0.254) (layer F.Cu) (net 5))
 (segment (start 28.66 19.924) (end 30.45 21.714) (width 0.254) (layer F.Cu) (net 5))
 (segment (start 30.45 21.714) (end 30.45 22.21) (width 0.254) (layer F.Cu) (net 5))
 (segment (start 28.66 17.88) (end 28.66 19.924) (width 0.254) (layer F.Cu) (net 5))
 (segment (start 34.26 16.38) (end 36.28 18.4) (width 0.254) (layer F.Cu) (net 6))
 (segment (start 28.66 16.38) (end 34.26 16.38) (width 0.254) (layer F.Cu) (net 6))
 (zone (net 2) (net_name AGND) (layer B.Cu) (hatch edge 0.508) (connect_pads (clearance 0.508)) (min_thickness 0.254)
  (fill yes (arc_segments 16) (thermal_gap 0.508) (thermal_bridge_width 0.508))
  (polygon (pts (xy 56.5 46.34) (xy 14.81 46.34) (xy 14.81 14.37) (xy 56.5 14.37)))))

